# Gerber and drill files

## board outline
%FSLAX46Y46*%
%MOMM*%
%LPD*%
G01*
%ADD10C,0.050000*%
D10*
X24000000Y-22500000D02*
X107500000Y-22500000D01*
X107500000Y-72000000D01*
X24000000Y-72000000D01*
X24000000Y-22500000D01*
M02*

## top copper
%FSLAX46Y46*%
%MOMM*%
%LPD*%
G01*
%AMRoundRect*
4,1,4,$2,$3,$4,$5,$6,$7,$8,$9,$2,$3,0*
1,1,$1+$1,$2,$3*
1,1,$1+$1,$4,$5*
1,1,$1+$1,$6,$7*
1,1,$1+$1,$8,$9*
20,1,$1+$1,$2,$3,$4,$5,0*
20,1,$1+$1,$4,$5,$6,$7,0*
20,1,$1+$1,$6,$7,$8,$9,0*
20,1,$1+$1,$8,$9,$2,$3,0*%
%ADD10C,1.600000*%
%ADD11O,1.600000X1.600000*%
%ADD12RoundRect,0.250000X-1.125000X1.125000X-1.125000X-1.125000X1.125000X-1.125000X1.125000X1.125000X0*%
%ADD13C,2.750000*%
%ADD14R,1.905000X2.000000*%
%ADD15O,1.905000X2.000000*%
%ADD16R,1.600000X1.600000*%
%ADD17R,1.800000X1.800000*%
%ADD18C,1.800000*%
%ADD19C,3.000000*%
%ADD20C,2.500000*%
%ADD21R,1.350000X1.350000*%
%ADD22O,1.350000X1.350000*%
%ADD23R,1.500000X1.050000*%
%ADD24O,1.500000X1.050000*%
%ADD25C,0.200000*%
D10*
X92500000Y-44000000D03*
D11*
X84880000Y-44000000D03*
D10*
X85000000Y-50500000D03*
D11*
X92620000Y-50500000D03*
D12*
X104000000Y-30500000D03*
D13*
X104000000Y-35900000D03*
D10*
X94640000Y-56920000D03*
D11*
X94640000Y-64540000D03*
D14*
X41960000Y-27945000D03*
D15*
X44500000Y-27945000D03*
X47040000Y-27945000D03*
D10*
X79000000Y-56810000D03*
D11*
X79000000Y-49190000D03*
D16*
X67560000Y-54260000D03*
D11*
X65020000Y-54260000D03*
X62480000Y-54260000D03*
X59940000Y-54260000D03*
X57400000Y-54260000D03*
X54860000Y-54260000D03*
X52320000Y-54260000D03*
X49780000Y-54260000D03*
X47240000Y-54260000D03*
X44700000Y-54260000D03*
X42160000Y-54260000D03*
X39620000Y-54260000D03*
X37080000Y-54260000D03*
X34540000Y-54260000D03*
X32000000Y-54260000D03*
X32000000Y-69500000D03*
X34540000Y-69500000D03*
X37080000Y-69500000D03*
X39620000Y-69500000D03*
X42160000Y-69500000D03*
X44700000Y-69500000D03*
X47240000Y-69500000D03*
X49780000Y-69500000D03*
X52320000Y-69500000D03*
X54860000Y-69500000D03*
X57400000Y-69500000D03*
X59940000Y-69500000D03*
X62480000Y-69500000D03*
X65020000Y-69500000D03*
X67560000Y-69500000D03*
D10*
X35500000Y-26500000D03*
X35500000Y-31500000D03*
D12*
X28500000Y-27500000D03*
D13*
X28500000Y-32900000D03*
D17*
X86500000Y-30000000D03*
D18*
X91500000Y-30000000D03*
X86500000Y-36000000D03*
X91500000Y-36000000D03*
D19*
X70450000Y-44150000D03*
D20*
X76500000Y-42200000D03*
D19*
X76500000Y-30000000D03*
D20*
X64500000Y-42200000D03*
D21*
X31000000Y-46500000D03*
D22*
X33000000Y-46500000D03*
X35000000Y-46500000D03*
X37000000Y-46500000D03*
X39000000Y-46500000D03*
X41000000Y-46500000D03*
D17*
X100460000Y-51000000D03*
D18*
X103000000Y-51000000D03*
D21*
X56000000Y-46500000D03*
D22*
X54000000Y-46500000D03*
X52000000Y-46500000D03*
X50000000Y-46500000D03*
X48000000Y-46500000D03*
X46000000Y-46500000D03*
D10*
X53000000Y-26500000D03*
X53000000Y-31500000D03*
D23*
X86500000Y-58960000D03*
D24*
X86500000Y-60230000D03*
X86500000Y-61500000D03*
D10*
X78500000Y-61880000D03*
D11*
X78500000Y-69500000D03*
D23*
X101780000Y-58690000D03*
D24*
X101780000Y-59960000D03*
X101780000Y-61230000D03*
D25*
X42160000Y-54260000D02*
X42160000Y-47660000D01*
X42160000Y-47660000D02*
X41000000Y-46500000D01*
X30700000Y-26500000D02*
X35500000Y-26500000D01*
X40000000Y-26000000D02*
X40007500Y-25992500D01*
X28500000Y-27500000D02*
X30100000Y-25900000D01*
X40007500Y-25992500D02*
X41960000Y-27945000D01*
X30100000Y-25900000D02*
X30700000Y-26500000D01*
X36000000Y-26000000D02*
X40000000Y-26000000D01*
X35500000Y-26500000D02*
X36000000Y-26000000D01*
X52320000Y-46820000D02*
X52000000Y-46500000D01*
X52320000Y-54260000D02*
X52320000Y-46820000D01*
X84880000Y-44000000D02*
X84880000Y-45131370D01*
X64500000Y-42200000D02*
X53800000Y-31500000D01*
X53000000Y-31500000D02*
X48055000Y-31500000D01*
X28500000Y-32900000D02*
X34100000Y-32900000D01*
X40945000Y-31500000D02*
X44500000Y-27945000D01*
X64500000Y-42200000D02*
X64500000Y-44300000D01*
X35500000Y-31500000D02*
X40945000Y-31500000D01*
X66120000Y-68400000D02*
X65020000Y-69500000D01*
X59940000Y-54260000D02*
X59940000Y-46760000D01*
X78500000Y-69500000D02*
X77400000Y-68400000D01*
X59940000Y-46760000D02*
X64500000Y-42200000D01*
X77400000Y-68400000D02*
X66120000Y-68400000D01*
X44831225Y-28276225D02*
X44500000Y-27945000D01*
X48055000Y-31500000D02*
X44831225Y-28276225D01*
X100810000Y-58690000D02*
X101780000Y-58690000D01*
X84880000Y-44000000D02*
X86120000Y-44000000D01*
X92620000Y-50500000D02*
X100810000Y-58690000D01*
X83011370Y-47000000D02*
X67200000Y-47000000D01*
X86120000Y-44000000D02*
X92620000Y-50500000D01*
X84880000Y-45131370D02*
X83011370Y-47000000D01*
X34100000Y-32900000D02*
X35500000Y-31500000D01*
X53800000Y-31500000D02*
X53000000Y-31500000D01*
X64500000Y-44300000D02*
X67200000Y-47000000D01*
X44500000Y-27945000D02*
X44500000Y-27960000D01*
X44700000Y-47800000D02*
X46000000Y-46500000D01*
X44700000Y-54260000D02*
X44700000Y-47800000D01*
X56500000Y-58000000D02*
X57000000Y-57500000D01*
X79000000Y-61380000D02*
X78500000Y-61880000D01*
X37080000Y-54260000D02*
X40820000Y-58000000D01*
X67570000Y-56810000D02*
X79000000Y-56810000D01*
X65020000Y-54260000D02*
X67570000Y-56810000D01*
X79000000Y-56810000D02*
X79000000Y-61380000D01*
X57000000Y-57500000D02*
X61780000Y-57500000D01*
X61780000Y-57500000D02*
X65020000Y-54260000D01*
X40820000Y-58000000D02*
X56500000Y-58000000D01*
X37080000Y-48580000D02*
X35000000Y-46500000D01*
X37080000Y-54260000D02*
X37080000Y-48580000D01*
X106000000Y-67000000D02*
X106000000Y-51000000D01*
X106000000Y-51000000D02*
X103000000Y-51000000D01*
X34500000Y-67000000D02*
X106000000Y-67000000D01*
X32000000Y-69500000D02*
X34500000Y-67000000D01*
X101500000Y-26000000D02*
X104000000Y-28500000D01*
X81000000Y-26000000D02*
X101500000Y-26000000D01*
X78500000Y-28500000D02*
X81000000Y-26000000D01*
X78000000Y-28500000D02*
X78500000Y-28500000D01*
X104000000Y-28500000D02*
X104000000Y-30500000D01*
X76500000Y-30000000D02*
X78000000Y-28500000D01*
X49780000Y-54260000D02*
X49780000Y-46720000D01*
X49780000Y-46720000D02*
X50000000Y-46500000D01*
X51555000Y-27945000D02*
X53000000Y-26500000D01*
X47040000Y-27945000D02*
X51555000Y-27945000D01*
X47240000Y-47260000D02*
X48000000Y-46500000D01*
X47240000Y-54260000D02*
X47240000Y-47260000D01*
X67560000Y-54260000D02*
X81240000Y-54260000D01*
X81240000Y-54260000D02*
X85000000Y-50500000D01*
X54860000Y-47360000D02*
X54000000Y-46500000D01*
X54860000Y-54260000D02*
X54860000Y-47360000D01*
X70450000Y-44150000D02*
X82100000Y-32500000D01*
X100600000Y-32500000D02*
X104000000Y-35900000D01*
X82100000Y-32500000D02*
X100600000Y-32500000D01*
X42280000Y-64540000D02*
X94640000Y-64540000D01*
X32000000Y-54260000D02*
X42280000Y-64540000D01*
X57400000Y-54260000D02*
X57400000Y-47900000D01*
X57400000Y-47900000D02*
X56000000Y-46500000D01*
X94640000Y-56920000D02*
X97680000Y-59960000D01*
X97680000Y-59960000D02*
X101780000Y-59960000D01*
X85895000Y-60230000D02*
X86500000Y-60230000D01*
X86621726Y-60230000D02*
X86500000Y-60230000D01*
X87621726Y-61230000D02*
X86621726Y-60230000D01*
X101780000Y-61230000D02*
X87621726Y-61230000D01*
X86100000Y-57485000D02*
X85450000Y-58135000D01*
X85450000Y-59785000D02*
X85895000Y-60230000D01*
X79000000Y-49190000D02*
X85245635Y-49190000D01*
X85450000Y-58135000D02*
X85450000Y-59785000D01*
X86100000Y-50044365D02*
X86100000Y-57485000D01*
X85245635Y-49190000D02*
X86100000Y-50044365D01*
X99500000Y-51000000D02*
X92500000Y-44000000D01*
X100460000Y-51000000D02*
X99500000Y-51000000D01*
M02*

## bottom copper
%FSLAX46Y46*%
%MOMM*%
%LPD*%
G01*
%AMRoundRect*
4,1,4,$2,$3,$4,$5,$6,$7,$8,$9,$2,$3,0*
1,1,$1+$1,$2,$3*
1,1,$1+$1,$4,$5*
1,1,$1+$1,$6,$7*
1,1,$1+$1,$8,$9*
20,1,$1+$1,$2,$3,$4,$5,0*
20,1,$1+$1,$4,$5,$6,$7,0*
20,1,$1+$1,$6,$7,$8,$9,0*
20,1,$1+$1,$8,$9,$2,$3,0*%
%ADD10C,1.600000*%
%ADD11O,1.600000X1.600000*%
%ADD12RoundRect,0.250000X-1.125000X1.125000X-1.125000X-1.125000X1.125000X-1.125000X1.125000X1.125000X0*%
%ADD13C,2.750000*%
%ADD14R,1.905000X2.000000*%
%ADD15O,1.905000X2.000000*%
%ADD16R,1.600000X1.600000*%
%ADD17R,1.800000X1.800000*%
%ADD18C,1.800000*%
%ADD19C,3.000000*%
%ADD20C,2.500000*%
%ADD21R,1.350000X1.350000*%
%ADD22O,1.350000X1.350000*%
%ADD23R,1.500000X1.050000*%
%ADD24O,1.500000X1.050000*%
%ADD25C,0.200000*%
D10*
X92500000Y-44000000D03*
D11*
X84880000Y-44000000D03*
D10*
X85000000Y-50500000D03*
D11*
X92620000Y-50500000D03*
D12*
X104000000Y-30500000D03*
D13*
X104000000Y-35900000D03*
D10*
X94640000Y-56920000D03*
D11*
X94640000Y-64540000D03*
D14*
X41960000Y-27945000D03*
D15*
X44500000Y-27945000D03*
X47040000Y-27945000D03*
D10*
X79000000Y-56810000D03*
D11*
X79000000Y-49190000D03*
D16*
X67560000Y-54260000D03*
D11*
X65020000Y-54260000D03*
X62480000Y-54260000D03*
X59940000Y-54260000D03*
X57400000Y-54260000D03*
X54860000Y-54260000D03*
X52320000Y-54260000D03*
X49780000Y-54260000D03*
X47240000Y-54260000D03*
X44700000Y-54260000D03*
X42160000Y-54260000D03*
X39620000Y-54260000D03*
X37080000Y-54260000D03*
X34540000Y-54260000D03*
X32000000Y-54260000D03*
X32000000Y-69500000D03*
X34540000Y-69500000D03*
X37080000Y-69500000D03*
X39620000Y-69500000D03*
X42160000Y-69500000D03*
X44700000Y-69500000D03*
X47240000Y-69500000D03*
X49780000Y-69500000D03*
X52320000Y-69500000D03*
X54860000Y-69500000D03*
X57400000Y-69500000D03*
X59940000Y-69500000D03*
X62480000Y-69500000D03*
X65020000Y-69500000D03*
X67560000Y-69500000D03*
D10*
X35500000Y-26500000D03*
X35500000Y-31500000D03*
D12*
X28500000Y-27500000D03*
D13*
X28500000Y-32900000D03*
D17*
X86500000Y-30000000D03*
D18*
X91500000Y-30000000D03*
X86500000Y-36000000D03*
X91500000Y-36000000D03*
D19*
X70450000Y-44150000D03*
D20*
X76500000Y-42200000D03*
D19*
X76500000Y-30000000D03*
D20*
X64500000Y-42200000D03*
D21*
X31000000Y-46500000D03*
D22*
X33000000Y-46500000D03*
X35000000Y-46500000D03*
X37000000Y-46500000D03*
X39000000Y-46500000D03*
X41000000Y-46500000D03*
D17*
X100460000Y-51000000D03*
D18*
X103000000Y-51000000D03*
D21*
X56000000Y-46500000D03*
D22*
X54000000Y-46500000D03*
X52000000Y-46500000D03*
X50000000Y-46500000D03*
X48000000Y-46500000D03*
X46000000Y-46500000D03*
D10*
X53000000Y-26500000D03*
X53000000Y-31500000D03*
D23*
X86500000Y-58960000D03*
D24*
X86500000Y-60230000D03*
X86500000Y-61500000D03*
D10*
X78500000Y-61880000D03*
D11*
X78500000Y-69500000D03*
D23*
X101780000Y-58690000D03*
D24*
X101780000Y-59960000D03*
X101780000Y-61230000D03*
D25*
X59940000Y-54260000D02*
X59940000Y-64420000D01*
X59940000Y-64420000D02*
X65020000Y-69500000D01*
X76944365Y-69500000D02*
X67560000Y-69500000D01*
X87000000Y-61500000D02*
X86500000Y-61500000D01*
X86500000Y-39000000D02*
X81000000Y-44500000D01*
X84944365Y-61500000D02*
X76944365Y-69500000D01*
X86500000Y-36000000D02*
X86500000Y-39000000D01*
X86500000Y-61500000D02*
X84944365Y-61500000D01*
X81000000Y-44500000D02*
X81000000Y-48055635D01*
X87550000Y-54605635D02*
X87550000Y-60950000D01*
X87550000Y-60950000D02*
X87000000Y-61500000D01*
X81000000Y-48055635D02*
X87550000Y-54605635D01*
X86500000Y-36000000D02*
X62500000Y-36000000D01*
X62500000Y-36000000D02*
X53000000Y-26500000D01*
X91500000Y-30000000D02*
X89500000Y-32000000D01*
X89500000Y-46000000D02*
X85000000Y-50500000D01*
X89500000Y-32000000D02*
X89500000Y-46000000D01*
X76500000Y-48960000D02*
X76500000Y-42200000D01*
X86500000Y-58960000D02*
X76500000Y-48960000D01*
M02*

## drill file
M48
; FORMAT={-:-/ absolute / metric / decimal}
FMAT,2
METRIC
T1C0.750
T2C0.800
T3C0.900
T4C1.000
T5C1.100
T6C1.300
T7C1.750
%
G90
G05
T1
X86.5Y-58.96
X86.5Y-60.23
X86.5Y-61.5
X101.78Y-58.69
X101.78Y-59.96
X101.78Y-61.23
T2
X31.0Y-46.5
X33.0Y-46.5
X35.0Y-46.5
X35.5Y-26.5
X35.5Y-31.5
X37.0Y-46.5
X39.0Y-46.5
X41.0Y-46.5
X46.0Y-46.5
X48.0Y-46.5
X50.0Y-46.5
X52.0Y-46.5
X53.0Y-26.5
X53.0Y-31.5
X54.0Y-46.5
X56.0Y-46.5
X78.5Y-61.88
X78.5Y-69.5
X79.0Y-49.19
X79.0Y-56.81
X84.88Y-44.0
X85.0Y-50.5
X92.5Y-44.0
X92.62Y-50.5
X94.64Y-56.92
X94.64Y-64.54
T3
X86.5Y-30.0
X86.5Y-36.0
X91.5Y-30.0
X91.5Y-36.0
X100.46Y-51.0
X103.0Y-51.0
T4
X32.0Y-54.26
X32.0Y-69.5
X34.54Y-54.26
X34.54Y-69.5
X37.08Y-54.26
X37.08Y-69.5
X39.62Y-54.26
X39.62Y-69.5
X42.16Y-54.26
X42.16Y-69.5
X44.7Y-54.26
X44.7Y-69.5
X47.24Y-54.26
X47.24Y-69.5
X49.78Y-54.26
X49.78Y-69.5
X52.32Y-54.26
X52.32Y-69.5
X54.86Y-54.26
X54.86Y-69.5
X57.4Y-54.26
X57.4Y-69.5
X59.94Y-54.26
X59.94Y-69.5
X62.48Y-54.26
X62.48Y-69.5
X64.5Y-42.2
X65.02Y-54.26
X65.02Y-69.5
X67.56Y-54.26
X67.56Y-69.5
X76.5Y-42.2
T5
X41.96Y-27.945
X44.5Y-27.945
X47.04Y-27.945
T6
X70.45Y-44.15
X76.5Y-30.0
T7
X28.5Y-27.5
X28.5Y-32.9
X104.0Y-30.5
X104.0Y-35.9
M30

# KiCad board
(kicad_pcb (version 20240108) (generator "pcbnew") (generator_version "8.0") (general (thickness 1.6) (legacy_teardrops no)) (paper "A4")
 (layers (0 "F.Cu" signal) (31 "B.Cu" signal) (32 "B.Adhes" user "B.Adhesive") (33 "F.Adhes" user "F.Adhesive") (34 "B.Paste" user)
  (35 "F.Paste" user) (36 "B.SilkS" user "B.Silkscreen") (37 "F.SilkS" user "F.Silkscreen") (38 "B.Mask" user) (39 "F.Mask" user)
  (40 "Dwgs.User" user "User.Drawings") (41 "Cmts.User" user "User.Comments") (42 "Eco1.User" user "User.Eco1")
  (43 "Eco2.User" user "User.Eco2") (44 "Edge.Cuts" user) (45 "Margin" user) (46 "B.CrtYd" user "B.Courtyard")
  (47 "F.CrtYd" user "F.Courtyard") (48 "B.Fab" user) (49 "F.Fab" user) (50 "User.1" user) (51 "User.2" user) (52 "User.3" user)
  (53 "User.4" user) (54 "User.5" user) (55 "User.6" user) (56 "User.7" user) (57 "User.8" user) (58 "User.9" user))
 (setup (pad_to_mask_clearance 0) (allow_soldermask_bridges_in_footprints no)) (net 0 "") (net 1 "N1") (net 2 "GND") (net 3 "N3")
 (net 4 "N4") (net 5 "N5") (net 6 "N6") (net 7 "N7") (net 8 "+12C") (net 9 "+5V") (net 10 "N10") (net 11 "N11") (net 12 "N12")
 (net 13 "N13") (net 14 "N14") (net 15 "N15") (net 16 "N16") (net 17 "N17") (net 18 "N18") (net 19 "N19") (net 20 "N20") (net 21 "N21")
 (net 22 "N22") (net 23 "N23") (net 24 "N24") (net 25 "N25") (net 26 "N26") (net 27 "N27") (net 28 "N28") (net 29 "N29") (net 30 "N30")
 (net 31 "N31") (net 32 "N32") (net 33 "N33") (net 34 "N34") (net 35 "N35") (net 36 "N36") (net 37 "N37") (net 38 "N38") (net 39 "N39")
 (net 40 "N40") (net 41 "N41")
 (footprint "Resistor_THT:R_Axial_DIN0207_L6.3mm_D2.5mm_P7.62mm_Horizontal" (layer "F.Cu") (at 92.5 44 180)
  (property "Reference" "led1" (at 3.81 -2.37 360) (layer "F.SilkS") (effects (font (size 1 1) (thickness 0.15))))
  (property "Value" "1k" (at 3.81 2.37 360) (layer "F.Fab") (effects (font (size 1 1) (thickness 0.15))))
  (pad "1" thru_hole circle (at 0 0 180) (size 1.6 1.6) (drill 0.8) (layers "*.Cu" "*.Mask") (remove_unused_layers no) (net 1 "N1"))
  (pad "2" thru_hole oval (at 7.62 0 180) (size 1.6 1.6) (drill 0.8) (layers "*.Cu" "*.Mask") (remove_unused_layers no) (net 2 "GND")))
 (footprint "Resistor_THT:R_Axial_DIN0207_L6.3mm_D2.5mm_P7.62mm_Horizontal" (layer "F.Cu") (at 85 50.5)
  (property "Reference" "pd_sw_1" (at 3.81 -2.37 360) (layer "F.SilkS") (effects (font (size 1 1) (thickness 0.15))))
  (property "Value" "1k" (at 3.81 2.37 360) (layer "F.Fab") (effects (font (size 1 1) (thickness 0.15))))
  (pad "1" thru_hole circle (at 0 0) (size 1.6 1.6) (drill 0.8) (layers "*.Cu" "*.Mask") (remove_unused_layers no) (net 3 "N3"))
  (pad "2" thru_hole oval (at 7.62 0) (size 1.6 1.6) (drill 0.8) (layers "*.Cu" "*.Mask") (remove_unused_layers no) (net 2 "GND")))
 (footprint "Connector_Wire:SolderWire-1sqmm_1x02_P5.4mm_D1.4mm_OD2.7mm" (layer "F.Cu") (at 104 30.5 -90)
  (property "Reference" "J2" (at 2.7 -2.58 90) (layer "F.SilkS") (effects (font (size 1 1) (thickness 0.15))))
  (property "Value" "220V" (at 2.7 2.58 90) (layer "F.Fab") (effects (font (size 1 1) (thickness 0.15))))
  (pad "1" thru_hole roundrect (at 0 0 270) (size 2.75 2.75) (drill 1.75) (layers "*.Cu" "*.Mask") (remove_unused_layers no)
   (roundrect_rratio 0.090909) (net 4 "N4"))
  (pad "2" thru_hole circle (at 5.4 0 270) (size 2.75 2.75) (drill 1.75) (layers "*.Cu" "*.Mask") (remove_unused_layers no) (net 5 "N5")))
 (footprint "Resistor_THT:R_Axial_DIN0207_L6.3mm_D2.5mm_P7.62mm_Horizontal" (layer "F.Cu") (at 94.64 56.92 -90)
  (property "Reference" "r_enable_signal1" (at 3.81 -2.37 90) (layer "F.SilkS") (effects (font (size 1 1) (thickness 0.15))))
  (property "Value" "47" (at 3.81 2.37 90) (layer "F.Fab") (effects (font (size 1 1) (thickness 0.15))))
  (pad "1" thru_hole circle (at 0 0 270) (size 1.6 1.6) (drill 0.8) (layers "*.Cu" "*.Mask") (remove_unused_layers no) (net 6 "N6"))
  (pad "2" thru_hole oval (at 7.62 0 270) (size 1.6 1.6) (drill 0.8) (layers "*.Cu" "*.Mask") (remove_unused_layers no) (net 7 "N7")))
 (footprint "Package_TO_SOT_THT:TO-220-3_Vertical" (layer "F.Cu") (at 41.96 27.945)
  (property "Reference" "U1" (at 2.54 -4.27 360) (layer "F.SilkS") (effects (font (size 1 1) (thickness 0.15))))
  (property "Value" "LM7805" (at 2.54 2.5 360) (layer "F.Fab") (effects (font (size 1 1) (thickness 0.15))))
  (pad "1" thru_hole rect (at 0 0) (size 1.905 2) (drill 1.1) (layers "*.Cu" "*.Mask") (remove_unused_layers no) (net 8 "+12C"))
  (pad "2" thru_hole oval (at 2.54 0) (size 1.905 2) (drill 1.1) (layers "*.Cu" "*.Mask") (remove_unused_layers no) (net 2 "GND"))
  (pad "3" thru_hole oval (at 5.08 0) (size 1.905 2) (drill 1.1) (layers "*.Cu" "*.Mask") (remove_unused_layers no) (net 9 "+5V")))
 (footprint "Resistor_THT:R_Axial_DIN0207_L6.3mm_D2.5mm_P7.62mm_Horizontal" (layer "F.Cu") (at 79 56.81 90)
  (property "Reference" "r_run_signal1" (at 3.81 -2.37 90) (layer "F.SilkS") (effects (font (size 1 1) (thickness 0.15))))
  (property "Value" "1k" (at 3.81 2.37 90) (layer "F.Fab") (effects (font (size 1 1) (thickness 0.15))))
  (pad "1" thru_hole circle (at 0 0 90) (size 1.6 1.6) (drill 0.8) (layers "*.Cu" "*.Mask") (remove_unused_layers no) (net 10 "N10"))
  (pad "2" thru_hole oval (at 7.62 0 90) (size 1.6 1.6) (drill 0.8) (layers "*.Cu" "*.Mask") (remove_unused_layers no) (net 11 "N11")))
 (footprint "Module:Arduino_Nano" (layer "F.Cu") (at 67.56 54.26 -90)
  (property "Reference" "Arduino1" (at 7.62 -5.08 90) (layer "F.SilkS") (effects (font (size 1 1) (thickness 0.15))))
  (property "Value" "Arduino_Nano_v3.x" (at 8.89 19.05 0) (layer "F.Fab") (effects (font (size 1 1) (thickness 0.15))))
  (pad "1" thru_hole rect (at 0 0 270) (size 1.6 1.6) (drill 1) (layers "*.Cu" "*.Mask") (remove_unused_layers no) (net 3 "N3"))
  (pad "2" thru_hole oval (at 0 2.54 270) (size 1.6 1.6) (drill 1) (layers "*.Cu" "*.Mask") (remove_unused_layers no) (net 10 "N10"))
  (pad "3" thru_hole oval (at 0 5.08 270) (size 1.6 1.6) (drill 1) (layers "*.Cu" "*.Mask") (remove_unused_layers no) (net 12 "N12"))
  (pad "4" thru_hole oval (at 0 7.62 270) (size 1.6 1.6) (drill 1) (layers "*.Cu" "*.Mask") (remove_unused_layers no) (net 2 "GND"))
  (pad "5" thru_hole oval (at 0 10.16 270) (size 1.6 1.6) (drill 1) (layers "*.Cu" "*.Mask") (remove_unused_layers no) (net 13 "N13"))
  (pad "6" thru_hole oval (at 0 12.7 270) (size 1.6 1.6) (drill 1) (layers "*.Cu" "*.Mask") (remove_unused_layers no) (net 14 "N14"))
  (pad "7" thru_hole oval (at 0 15.24 270) (size 1.6 1.6) (drill 1) (layers "*.Cu" "*.Mask") (remove_unused_layers no) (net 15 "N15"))
  (pad "8" thru_hole oval (at 0 17.78 270) (size 1.6 1.6) (drill 1) (layers "*.Cu" "*.Mask") (remove_unused_layers no) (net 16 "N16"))
  (pad "9" thru_hole oval (at 0 20.32 270) (size 1.6 1.6) (drill 1) (layers "*.Cu" "*.Mask") (remove_unused_layers no) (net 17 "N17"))
  (pad "10" thru_hole oval (at 0 22.86 270) (size 1.6 1.6) (drill 1) (layers "*.Cu" "*.Mask") (remove_unused_layers no) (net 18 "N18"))
  (pad "11" thru_hole oval (at 0 25.4 270) (size 1.6 1.6) (drill 1) (layers "*.Cu" "*.Mask") (remove_unused_layers no) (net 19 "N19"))
  (pad "12" thru_hole oval (at 0 27.94 270) (size 1.6 1.6) (drill 1) (layers "*.Cu" "*.Mask") (remove_unused_layers no) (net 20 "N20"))
  (pad "13" thru_hole oval (at 0 30.48 270) (size 1.6 1.6) (drill 1) (layers "*.Cu" "*.Mask") (remove_unused_layers no) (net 10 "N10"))
  (pad "14" thru_hole oval (at 0 33.02 270) (size 1.6 1.6) (drill 1) (layers "*.Cu" "*.Mask") (remove_unused_layers no) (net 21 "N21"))
  (pad "15" thru_hole oval (at 0 35.56 270) (size 1.6 1.6) (drill 1) (layers "*.Cu" "*.Mask") (remove_unused_layers no) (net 7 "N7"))
  (pad "16" thru_hole oval (at 15.24 35.56 270) (size 1.6 1.6) (drill 1) (layers "*.Cu" "*.Mask") (remove_unused_layers no) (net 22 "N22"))
  (pad "17" thru_hole oval (at 15.24 33.02 270) (size 1.6 1.6) (drill 1) (layers "*.Cu" "*.Mask") (remove_unused_layers no) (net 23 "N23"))
  (pad "18" thru_hole oval (at 15.24 30.48 270) (size 1.6 1.6) (drill 1) (layers "*.Cu" "*.Mask") (remove_unused_layers no) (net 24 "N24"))
  (pad "19" thru_hole oval (at 15.24 27.94 270) (size 1.6 1.6) (drill 1) (layers "*.Cu" "*.Mask") (remove_unused_layers no) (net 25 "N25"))
  (pad "20" thru_hole oval (at 15.24 25.4 270) (size 1.6 1.6) (drill 1) (layers "*.Cu" "*.Mask") (remove_unused_layers no) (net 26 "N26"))
  (pad "21" thru_hole oval (at 15.24 22.86 270) (size 1.6 1.6) (drill 1) (layers "*.Cu" "*.Mask") (remove_unused_layers no) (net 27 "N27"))
  (pad "22" thru_hole oval (at 15.24 20.32 270) (size 1.6 1.6) (drill 1) (layers "*.Cu" "*.Mask") (remove_unused_layers no) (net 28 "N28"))
  (pad "23" thru_hole oval (at 15.24 17.78 270) (size 1.6 1.6) (drill 1) (layers "*.Cu" "*.Mask") (remove_unused_layers no) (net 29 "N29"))
  (pad "24" thru_hole oval (at 15.24 15.24 270) (size 1.6 1.6) (drill 1) (layers "*.Cu" "*.Mask") (remove_unused_layers no) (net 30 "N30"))
  (pad "25" thru_hole oval (at 15.24 12.7 270) (size 1.6 1.6) (drill 1) (layers "*.Cu" "*.Mask") (remove_unused_layers no) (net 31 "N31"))
  (pad "26" thru_hole oval (at 15.24 10.16 270) (size 1.6 1.6) (drill 1) (layers "*.Cu" "*.Mask") (remove_unused_layers no) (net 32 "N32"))
  (pad "27" thru_hole oval (at 15.24 7.62 270) (size 1.6 1.6) (drill 1) (layers "*.Cu" "*.Mask") (remove_unused_layers no) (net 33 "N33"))
  (pad "28" thru_hole oval (at 15.24 5.08 270) (size 1.6 1.6) (drill 1) (layers "*.Cu" "*.Mask") (remove_unused_layers no) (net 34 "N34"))
  (pad "29" thru_hole oval (at 15.24 2.54 270) (size 1.6 1.6) (drill 1) (layers "*.Cu" "*.Mask") (remove_unused_layers no) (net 2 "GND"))
  (pad "30" thru_hole oval (at 15.24 0 270) (size 1.6 1.6) (drill 1) (layers "*.Cu" "*.Mask") (remove_unused_layers no) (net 9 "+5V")))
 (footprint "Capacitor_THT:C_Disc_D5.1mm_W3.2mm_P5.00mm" (layer "F.Cu") (at 35.5 26.5 -90)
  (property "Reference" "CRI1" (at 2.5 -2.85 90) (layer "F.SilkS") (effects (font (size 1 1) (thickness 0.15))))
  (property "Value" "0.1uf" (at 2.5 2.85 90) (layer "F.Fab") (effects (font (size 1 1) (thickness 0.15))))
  (pad "1" thru_hole circle (at 0 0 270) (size 1.6 1.6) (drill 0.8) (layers "*.Cu" "*.Mask") (remove_unused_layers no) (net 8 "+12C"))
  (pad "2" thru_hole circle (at 5 0 270) (size 1.6 1.6) (drill 0.8) (layers "*.Cu" "*.Mask") (remove_unused_layers no) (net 2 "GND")))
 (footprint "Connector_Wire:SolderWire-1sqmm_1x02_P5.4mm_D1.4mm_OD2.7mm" (layer "F.Cu") (at 28.5 27.5 -90)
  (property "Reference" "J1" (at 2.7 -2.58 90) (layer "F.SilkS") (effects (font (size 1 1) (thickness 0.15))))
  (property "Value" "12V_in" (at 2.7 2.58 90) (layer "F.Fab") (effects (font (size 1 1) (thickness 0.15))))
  (pad "1" thru_hole roundrect (at 0 0 270) (size 2.75 2.75) (drill 1.75) (layers "*.Cu" "*.Mask") (remove_unused_layers no)
   (roundrect_rratio 0.090909) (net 8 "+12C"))
  (pad "2" thru_hole circle (at 5.4 0 270) (size 2.75 2.75) (drill 1.75) (layers "*.Cu" "*.Mask") (remove_unused_layers no) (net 2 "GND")))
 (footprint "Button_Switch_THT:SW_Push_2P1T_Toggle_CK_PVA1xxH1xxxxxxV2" (layer "F.Cu") (at 86.5 30)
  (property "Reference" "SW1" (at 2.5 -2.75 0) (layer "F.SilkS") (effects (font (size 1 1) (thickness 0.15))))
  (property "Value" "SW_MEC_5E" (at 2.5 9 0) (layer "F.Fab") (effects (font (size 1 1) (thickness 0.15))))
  (pad "1" thru_hole rect (at 0 0) (size 1.8 1.8) (drill 0.9) (layers "*.Cu" "*.Mask") (remove_unused_layers no) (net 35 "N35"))
  (pad "2" thru_hole circle (at 5 0) (size 1.8 1.8) (drill 0.9) (layers "*.Cu" "*.Mask") (remove_unused_layers no) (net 3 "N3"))
  (pad "3" thru_hole circle (at 0 6) (size 1.8 1.8) (drill 0.9) (layers "*.Cu" "*.Mask") (remove_unused_layers no) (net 9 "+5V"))
  (pad "4" thru_hole circle (at 5 6) (size 1.8 1.8) (drill 0.9) (layers "*.Cu" "*.Mask") (remove_unused_layers no) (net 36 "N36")))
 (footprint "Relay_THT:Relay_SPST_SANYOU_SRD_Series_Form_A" (layer "F.Cu") (at 70.45 44.15 90)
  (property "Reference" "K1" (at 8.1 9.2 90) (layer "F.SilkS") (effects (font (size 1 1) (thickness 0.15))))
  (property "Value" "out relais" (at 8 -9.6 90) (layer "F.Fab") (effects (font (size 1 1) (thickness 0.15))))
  (pad "1" thru_hole circle (at 0 0 180) (size 3 3) (drill 1.3) (layers "*.Cu" "*.Mask") (remove_unused_layers no) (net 5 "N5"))
  (pad "2" thru_hole circle (at 1.95 6.05 180) (size 2.5 2.5) (drill 1) (layers "*.Cu" "*.Mask") (remove_unused_layers no) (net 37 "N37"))
  (pad "3" thru_hole circle (at 14.15 6.05 180) (size 3 3) (drill 1.3) (layers "*.Cu" "*.Mask") (remove_unused_layers no) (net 4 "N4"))
  (pad "5" thru_hole circle (at 1.95 -5.95 180) (size 2.5 2.5) (drill 1) (layers "*.Cu" "*.Mask") (remove_unused_layers no) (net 2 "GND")))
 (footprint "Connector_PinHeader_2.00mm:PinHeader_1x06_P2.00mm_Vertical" (layer "F.Cu") (at 31 46.5 90)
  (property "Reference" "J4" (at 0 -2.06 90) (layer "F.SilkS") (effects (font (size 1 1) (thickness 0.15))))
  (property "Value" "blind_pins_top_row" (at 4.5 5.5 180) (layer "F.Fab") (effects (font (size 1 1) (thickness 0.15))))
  (pad "1" thru_hole rect (at 0 0 90) (size 1.35 1.35) (drill 0.8) (layers "*.Cu" "*.Mask") (remove_unused_layers no) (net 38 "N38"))
  (pad "2" thru_hole oval (at 0 2 90) (size 1.35 1.35) (drill 0.8) (layers "*.Cu" "*.Mask") (remove_unused_layers no) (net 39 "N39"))
  (pad "3" thru_hole oval (at 0 4 90) (size 1.35 1.35) (drill 0.8) (layers "*.Cu" "*.Mask") (remove_unused_layers no) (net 10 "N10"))
  (pad "4" thru_hole oval (at 0 6 90) (size 1.35 1.35) (drill 0.8) (layers "*.Cu" "*.Mask") (remove_unused_layers no) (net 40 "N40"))
  (pad "5" thru_hole oval (at 0 8 90) (size 1.35 1.35) (drill 0.8) (layers "*.Cu" "*.Mask") (remove_unused_layers no) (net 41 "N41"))
  (pad "6" thru_hole oval (at 0 10 90) (size 1.35 1.35) (drill 0.8) (layers "*.Cu" "*.Mask") (remove_unused_layers no) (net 19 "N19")))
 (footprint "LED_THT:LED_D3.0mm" (layer "F.Cu") (at 100.46 51)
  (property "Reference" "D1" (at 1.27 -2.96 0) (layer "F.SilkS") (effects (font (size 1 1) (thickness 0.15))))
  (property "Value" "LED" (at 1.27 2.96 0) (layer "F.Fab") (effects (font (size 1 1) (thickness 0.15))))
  (pad "1" thru_hole rect (at 0 0) (size 1.8 1.8) (drill 0.9) (layers "*.Cu" "*.Mask") (remove_unused_layers no) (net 1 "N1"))
  (pad "2" thru_hole circle (at 2.54 0) (size 1.8 1.8) (drill 0.9) (layers "*.Cu" "*.Mask") (remove_unused_layers no) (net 22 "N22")))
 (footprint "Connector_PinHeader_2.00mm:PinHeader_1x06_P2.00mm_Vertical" (layer "F.Cu") (at 56 46.5 -90)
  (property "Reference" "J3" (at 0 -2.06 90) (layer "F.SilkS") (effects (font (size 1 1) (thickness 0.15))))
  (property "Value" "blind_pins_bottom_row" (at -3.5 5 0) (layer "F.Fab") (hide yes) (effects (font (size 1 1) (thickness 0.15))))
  (pad "1" thru_hole rect (at 0 0 270) (size 1.35 1.35) (drill 0.8) (layers "*.Cu" "*.Mask") (remove_unused_layers no) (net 13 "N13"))
  (pad "2" thru_hole oval (at 0 2 270) (size 1.35 1.35) (drill 0.8) (layers "*.Cu" "*.Mask") (remove_unused_layers no) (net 14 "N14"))
  (pad "3" thru_hole oval (at 0 4 270) (size 1.35 1.35) (drill 0.8) (layers "*.Cu" "*.Mask") (remove_unused_layers no) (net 15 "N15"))
  (pad "4" thru_hole oval (at 0 6 270) (size 1.35 1.35) (drill 0.8) (layers "*.Cu" "*.Mask") (remove_unused_layers no) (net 16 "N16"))
  (pad "5" thru_hole oval (at 0 8 270) (size 1.35 1.35) (drill 0.8) (layers "*.Cu" "*.Mask") (remove_unused_layers no) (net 17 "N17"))
  (pad "6" thru_hole oval (at 0 10 270) (size 1.35 1.35) (drill 0.8) (layers "*.Cu" "*.Mask") (remove_unused_layers no) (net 18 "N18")))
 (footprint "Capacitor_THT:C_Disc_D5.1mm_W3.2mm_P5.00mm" (layer "F.Cu") (at 53 26.5 -90)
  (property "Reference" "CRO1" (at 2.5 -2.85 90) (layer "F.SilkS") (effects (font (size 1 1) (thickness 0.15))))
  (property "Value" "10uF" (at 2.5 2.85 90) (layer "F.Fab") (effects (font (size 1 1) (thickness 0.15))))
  (pad "1" thru_hole circle (at 0 0 270) (size 1.6 1.6) (drill 0.8) (layers "*.Cu" "*.Mask") (remove_unused_layers no) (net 9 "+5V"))
  (pad "2" thru_hole circle (at 5 0 270) (size 1.6 1.6) (drill 0.8) (layers "*.Cu" "*.Mask") (remove_unused_layers no) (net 2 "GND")))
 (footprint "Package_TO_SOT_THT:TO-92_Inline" (layer "F.Cu") (at 86.5 58.96 -90)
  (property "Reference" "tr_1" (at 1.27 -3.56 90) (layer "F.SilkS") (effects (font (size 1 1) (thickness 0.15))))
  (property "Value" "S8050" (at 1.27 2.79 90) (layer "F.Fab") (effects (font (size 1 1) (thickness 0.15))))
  (pad "1" thru_hole rect (at 0 0 270) (size 1.05 1.5) (drill 0.75) (layers "*.Cu" "*.Mask") (remove_unused_layers no) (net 37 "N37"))
  (pad "2" thru_hole oval (at 1.27 0 270) (size 1.05 1.5) (drill 0.75) (layers "*.Cu" "*.Mask") (remove_unused_layers no) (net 11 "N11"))
  (pad "3" thru_hole oval (at 2.54 0 270) (size 1.05 1.5) (drill 0.75) (layers "*.Cu" "*.Mask") (remove_unused_layers no) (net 9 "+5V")))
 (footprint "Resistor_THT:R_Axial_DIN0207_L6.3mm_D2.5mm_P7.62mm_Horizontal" (layer "F.Cu") (at 78.5 61.88 -90)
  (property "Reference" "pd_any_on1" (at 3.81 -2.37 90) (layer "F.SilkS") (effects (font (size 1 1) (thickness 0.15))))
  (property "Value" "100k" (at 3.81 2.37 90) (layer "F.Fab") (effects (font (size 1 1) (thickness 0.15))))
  (pad "1" thru_hole circle (at 0 0 270) (size 1.6 1.6) (drill 0.8) (layers "*.Cu" "*.Mask") (remove_unused_layers no) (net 10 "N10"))
  (pad "2" thru_hole oval (at 7.62 0 270) (size 1.6 1.6) (drill 0.8) (layers "*.Cu" "*.Mask") (remove_unused_layers no) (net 2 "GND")))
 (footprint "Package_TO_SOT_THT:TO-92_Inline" (layer "F.Cu") (at 101.78 58.69 -90)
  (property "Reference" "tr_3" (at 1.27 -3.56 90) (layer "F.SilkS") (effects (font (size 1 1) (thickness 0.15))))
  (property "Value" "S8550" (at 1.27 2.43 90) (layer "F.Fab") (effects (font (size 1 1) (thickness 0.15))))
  (pad "1" thru_hole rect (at 0 0 270) (size 1.05 1.5) (drill 0.75) (layers "*.Cu" "*.Mask") (remove_unused_layers no) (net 2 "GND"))
  (pad "2" thru_hole oval (at 1.27 0 270) (size 1.05 1.5) (drill 0.75) (layers "*.Cu" "*.Mask") (remove_unused_layers no) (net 6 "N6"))
  (pad "3" thru_hole oval (at 2.54 0 270) (size 1.05 1.5) (drill 0.75) (layers "*.Cu" "*.Mask") (remove_unused_layers no) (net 11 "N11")))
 (gr_rect (start 24 22.5) (end 107.5 72) (stroke (width 0.05) (type default)) (fill none) (layer "Edge.Cuts"))
 (segment (start 42.16 54.26) (end 42.16 47.66) (width 0.2) (layer "F.Cu") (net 19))
 (segment (start 42.16 47.66) (end 41 46.5) (width 0.2) (layer "F.Cu") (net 19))
 (segment (start 30.7 26.5) (end 35.5 26.5) (width 0.2) (layer "F.Cu") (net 8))
 (segment (start 40 26) (end 40.0075 25.9925) (width 0.2) (layer "F.Cu") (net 8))
 (segment (start 28.5 27.5) (end 30.1 25.9) (width 0.2) (layer "F.Cu") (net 8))
 (segment (start 40.0075 25.9925) (end 41.96 27.945) (width 0.2) (layer "F.Cu") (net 8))
 (segment (start 30.1 25.9) (end 30.7 26.5) (width 0.2) (layer "F.Cu") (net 8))
 (segment (start 36 26) (end 40 26) (width 0.2) (layer "F.Cu") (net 8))
 (segment (start 35.5 26.5) (end 36 26) (width 0.2) (layer "F.Cu") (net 8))
 (segment (start 52.32 46.82) (end 52 46.5) (width 0.2) (layer "F.Cu") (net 15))
 (segment (start 52.32 54.26) (end 52.32 46.82) (width 0.2) (layer "F.Cu") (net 15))
 (segment (start 84.88 44) (end 84.88 45.13137) (width 0.2) (layer "F.Cu") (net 2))
 (segment (start 64.5 42.2) (end 53.8 31.5) (width 0.2) (layer "F.Cu") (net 2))
 (segment (start 53 31.5) (end 48.055 31.5) (width 0.2) (layer "F.Cu") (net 2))
 (segment (start 28.5 32.9) (end 34.1 32.9) (width 0.2) (layer "F.Cu") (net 2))
 (segment (start 40.945 31.5) (end 44.5 27.945) (width 0.2) (layer "F.Cu") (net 2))
 (segment (start 64.5 42.2) (end 64.5 44.3) (width 0.2) (layer "F.Cu") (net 2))
 (segment (start 35.5 31.5) (end 40.945 31.5) (width 0.2) (layer "F.Cu") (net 2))
 (segment (start 66.12 68.4) (end 65.02 69.5) (width 0.2) (layer "F.Cu") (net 2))
 (segment (start 59.94 54.26) (end 59.94 46.76) (width 0.2) (layer "F.Cu") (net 2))
 (segment (start 78.5 69.5) (end 77.4 68.4) (width 0.2) (layer "F.Cu") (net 2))
 (segment (start 59.94 46.76) (end 64.5 42.2) (width 0.2) (layer "F.Cu") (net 2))
 (segment (start 77.4 68.4) (end 66.12 68.4) (width 0.2) (layer "F.Cu") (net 2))
 (segment (start 44.831225 28.276225) (end 44.5 27.945) (width 0.2) (layer "F.Cu") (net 2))
 (segment (start 48.055 31.5) (end 44.831225 28.276225) (width 0.2) (layer "F.Cu") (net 2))
 (segment (start 100.81 58.69) (end 101.78 58.69) (width 0.2) (layer "F.Cu") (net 2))
 (segment (start 84.88 44) (end 86.12 44) (width 0.2) (layer "F.Cu") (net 2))
 (segment (start 92.62 50.5) (end 100.81 58.69) (width 0.2) (layer "F.Cu") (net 2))
 (segment (start 83.01137 47) (end 67.2 47) (width 0.2) (layer "F.Cu") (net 2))
 (segment (start 86.12 44) (end 92.62 50.5) (width 0.2) (layer "F.Cu") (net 2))
 (segment (start 84.88 45.13137) (end 83.01137 47) (width 0.2) (layer "F.Cu") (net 2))
 (segment (start 34.1 32.9) (end 35.5 31.5) (width 0.2) (layer "F.Cu") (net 2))
 (segment (start 53.8 31.5) (end 53 31.5) (width 0.2) (layer "F.Cu") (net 2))
 (segment (start 64.5 44.3) (end 67.2 47) (width 0.2) (layer "F.Cu") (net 2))
 (segment (start 44.5 27.945) (end 44.5 27.96) (width 0.2) (layer "F.Cu") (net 2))
 (segment (start 59.94 54.26) (end 59.94 64.42) (width 0.2) (layer "B.Cu") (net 2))
 (segment (start 59.94 64.42) (end 65.02 69.5) (width 0.2) (layer "B.Cu") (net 2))
 (segment (start 44.7 47.8) (end 46 46.5) (width 0.2) (layer "F.Cu") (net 18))
 (segment (start 44.7 54.26) (end 44.7 47.8) (width 0.2) (layer "F.Cu") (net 18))
 (segment (start 56.5 58) (end 57 57.5) (width 0.2) (layer "F.Cu") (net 10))
 (segment (start 79 61.38) (end 78.5 61.88) (width 0.2) (layer "F.Cu") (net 10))
 (segment (start 37.08 54.26) (end 40.82 58) (width 0.2) (layer "F.Cu") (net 10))
 (segment (start 67.57 56.81) (end 79 56.81) (width 0.2) (layer "F.Cu") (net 10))
 (segment (start 65.02 54.26) (end 67.57 56.81) (width 0.2) (layer "F.Cu") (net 10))
 (segment (start 79 56.81) (end 79 61.38) (width 0.2) (layer "F.Cu") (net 10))
 (segment (start 57 57.5) (end 61.78 57.5) (width 0.2) (layer "F.Cu") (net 10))
 (segment (start 61.78 57.5) (end 65.02 54.26) (width 0.2) (layer "F.Cu") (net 10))
 (segment (start 40.82 58) (end 56.5 58) (width 0.2) (layer "F.Cu") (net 10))
 (segment (start 37.08 48.58) (end 35 46.5) (width 0.2) (layer "F.Cu") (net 10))
 (segment (start 37.08 54.26) (end 37.08 48.58) (width 0.2) (layer "F.Cu") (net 10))
 (segment (start 106 67) (end 106 51) (width 0.2) (layer "F.Cu") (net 22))
 (segment (start 106 51) (end 103 51) (width 0.2) (layer "F.Cu") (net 22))
 (segment (start 34.5 67) (end 106 67) (width 0.2) (layer "F.Cu") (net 22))
 (segment (start 32 69.5) (end 34.5 67) (width 0.2) (layer "F.Cu") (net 22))
 (segment (start 101.5 26) (end 104 28.5) (width 0.2) (layer "F.Cu") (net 4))
 (segment (start 81 26) (end 101.5 26) (width 0.2) (layer "F.Cu") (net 4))
 (segment (start 78.5 28.5) (end 81 26) (width 0.2) (layer "F.Cu") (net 4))
 (segment (start 78 28.5) (end 78.5 28.5) (width 0.2) (layer "F.Cu") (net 4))
 (segment (start 104 28.5) (end 104 30.5) (width 0.2) (layer "F.Cu") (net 4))
 (segment (start 76.5 30) (end 78 28.5) (width 0.2) (layer "F.Cu") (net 4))
 (segment (start 49.78 54.26) (end 49.78 46.72) (width 0.2) (layer "F.Cu") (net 16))
 (segment (start 49.78 46.72) (end 50 46.5) (width 0.2) (layer "F.Cu") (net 16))
 (segment (start 51.555 27.945) (end 53 26.5) (width 0.2) (layer "F.Cu") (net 9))
 (segment (start 47.04 27.945) (end 51.555 27.945) (width 0.2) (layer "F.Cu") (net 9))
 (segment (start 76.944365 69.5) (end 67.56 69.5) (width 0.2) (layer "B.Cu") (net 9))
 (segment (start 87 61.5) (end 86.5 61.5) (width 0.2) (layer "B.Cu") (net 9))
 (segment (start 86.5 39) (end 81 44.5) (width 0.2) (layer "B.Cu") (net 9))
 (segment (start 84.944365 61.5) (end 76.944365 69.5) (width 0.2) (layer "B.Cu") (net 9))
 (segment (start 86.5 36) (end 86.5 39) (width 0.2) (layer "B.Cu") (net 9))
 (segment (start 86.5 61.5) (end 84.944365 61.5) (width 0.2) (layer "B.Cu") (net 9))
 (segment (start 81 44.5) (end 81 48.055635) (width 0.2) (layer "B.Cu") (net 9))
 (segment (start 87.55 54.605635) (end 87.55 60.95) (width 0.2) (layer "B.Cu") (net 9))
 (segment (start 87.55 60.95) (end 87 61.5) (width 0.2) (layer "B.Cu") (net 9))
 (segment (start 81 48.055635) (end 87.55 54.605635) (width 0.2) (layer "B.Cu") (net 9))
 (segment (start 86.5 36) (end 62.5 36) (width 0.2) (layer "B.Cu") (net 9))
 (segment (start 62.5 36) (end 53 26.5) (width 0.2) (layer "B.Cu") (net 9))
 (segment (start 47.24 47.26) (end 48 46.5) (width 0.2) (layer "F.Cu") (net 17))
 (segment (start 47.24 54.26) (end 47.24 47.26) (width 0.2) (layer "F.Cu") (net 17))
 (segment (start 67.56 54.26) (end 81.24 54.26) (width 0.2) (layer "F.Cu") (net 3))
 (segment (start 81.24 54.26) (end 85 50.5) (width 0.2) (layer "F.Cu") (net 3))
 (segment (start 91.5 30) (end 89.5 32) (width 0.2) (layer "B.Cu") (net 3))
 (segment (start 89.5 46) (end 85 50.5) (width 0.2) (layer "B.Cu") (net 3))
 (segment (start 89.5 32) (end 89.5 46) (width 0.2) (layer "B.Cu") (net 3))
 (segment (start 54.86 47.36) (end 54 46.5) (width 0.2) (layer "F.Cu") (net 14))
 (segment (start 54.86 54.26) (end 54.86 47.36) (width 0.2) (layer "F.Cu") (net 14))
 (segment (start 70.45 44.15) (end 82.1 32.5) (width 0.2) (layer "F.Cu") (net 5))
 (segment (start 100.6 32.5) (end 104 35.9) (width 0.2) (layer "F.Cu") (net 5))
 (segment (start 82.1 32.5) (end 100.6 32.5) (width 0.2) (layer "F.Cu") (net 5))
 (segment (start 42.28 64.54) (end 94.64 64.54) (width 0.2) (layer "F.Cu") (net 7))
 (segment (start 32 54.26) (end 42.28 64.54) (width 0.2) (layer "F.Cu") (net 7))
 (segment (start 57.4 54.26) (end 57.4 47.9) (width 0.2) (layer "F.Cu") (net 13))
 (segment (start 57.4 47.9) (end 56 46.5) (width 0.2) (layer "F.Cu") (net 13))
 (segment (start 94.64 56.92) (end 97.68 59.96) (width 0.2) (layer "F.Cu") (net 6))
 (segment (start 97.68 59.96) (end 101.78 59.96) (width 0.2) (layer "F.Cu") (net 6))
 (segment (start 85.895 60.23) (end 86.5 60.23) (width 0.2) (layer "F.Cu") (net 11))
 (segment (start 86.621726 60.23) (end 86.5 60.23) (width 0.2) (layer "F.Cu") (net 11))
 (segment (start 87.621726 61.23) (end 86.621726 60.23) (width 0.2) (layer "F.Cu") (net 11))
 (segment (start 101.78 61.23) (end 87.621726 61.23) (width 0.2) (layer "F.Cu") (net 11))
 (segment (start 86.1 57.485) (end 85.45 58.135) (width 0.2) (layer "F.Cu") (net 11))
 (segment (start 85.45 59.785) (end 85.895 60.23) (width 0.2) (layer "F.Cu") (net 11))
 (segment (start 79 49.19) (end 85.245635 49.19) (width 0.2) (layer "F.Cu") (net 11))
 (segment (start 85.45 58.135) (end 85.45 59.785) (width 0.2) (layer "F.Cu") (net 11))
 (segment (start 86.1 50.044365) (end 86.1 57.485) (width 0.2) (layer "F.Cu") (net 11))
 (segment (start 85.245635 49.19) (end 86.1 50.044365) (width 0.2) (layer "F.Cu") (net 11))
 (segment (start 76.5 48.96) (end 76.5 42.2) (width 0.2) (layer "B.Cu") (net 37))
 (segment (start 86.5 58.96) (end 76.5 48.96) (width 0.2) (layer "B.Cu") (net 37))
 (segment (start 99.5 51) (end 92.5 44) (width 0.2) (layer "F.Cu") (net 1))
 (segment (start 100.46 51) (end 99.5 51) (width 0.2) (layer "F.Cu") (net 1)))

